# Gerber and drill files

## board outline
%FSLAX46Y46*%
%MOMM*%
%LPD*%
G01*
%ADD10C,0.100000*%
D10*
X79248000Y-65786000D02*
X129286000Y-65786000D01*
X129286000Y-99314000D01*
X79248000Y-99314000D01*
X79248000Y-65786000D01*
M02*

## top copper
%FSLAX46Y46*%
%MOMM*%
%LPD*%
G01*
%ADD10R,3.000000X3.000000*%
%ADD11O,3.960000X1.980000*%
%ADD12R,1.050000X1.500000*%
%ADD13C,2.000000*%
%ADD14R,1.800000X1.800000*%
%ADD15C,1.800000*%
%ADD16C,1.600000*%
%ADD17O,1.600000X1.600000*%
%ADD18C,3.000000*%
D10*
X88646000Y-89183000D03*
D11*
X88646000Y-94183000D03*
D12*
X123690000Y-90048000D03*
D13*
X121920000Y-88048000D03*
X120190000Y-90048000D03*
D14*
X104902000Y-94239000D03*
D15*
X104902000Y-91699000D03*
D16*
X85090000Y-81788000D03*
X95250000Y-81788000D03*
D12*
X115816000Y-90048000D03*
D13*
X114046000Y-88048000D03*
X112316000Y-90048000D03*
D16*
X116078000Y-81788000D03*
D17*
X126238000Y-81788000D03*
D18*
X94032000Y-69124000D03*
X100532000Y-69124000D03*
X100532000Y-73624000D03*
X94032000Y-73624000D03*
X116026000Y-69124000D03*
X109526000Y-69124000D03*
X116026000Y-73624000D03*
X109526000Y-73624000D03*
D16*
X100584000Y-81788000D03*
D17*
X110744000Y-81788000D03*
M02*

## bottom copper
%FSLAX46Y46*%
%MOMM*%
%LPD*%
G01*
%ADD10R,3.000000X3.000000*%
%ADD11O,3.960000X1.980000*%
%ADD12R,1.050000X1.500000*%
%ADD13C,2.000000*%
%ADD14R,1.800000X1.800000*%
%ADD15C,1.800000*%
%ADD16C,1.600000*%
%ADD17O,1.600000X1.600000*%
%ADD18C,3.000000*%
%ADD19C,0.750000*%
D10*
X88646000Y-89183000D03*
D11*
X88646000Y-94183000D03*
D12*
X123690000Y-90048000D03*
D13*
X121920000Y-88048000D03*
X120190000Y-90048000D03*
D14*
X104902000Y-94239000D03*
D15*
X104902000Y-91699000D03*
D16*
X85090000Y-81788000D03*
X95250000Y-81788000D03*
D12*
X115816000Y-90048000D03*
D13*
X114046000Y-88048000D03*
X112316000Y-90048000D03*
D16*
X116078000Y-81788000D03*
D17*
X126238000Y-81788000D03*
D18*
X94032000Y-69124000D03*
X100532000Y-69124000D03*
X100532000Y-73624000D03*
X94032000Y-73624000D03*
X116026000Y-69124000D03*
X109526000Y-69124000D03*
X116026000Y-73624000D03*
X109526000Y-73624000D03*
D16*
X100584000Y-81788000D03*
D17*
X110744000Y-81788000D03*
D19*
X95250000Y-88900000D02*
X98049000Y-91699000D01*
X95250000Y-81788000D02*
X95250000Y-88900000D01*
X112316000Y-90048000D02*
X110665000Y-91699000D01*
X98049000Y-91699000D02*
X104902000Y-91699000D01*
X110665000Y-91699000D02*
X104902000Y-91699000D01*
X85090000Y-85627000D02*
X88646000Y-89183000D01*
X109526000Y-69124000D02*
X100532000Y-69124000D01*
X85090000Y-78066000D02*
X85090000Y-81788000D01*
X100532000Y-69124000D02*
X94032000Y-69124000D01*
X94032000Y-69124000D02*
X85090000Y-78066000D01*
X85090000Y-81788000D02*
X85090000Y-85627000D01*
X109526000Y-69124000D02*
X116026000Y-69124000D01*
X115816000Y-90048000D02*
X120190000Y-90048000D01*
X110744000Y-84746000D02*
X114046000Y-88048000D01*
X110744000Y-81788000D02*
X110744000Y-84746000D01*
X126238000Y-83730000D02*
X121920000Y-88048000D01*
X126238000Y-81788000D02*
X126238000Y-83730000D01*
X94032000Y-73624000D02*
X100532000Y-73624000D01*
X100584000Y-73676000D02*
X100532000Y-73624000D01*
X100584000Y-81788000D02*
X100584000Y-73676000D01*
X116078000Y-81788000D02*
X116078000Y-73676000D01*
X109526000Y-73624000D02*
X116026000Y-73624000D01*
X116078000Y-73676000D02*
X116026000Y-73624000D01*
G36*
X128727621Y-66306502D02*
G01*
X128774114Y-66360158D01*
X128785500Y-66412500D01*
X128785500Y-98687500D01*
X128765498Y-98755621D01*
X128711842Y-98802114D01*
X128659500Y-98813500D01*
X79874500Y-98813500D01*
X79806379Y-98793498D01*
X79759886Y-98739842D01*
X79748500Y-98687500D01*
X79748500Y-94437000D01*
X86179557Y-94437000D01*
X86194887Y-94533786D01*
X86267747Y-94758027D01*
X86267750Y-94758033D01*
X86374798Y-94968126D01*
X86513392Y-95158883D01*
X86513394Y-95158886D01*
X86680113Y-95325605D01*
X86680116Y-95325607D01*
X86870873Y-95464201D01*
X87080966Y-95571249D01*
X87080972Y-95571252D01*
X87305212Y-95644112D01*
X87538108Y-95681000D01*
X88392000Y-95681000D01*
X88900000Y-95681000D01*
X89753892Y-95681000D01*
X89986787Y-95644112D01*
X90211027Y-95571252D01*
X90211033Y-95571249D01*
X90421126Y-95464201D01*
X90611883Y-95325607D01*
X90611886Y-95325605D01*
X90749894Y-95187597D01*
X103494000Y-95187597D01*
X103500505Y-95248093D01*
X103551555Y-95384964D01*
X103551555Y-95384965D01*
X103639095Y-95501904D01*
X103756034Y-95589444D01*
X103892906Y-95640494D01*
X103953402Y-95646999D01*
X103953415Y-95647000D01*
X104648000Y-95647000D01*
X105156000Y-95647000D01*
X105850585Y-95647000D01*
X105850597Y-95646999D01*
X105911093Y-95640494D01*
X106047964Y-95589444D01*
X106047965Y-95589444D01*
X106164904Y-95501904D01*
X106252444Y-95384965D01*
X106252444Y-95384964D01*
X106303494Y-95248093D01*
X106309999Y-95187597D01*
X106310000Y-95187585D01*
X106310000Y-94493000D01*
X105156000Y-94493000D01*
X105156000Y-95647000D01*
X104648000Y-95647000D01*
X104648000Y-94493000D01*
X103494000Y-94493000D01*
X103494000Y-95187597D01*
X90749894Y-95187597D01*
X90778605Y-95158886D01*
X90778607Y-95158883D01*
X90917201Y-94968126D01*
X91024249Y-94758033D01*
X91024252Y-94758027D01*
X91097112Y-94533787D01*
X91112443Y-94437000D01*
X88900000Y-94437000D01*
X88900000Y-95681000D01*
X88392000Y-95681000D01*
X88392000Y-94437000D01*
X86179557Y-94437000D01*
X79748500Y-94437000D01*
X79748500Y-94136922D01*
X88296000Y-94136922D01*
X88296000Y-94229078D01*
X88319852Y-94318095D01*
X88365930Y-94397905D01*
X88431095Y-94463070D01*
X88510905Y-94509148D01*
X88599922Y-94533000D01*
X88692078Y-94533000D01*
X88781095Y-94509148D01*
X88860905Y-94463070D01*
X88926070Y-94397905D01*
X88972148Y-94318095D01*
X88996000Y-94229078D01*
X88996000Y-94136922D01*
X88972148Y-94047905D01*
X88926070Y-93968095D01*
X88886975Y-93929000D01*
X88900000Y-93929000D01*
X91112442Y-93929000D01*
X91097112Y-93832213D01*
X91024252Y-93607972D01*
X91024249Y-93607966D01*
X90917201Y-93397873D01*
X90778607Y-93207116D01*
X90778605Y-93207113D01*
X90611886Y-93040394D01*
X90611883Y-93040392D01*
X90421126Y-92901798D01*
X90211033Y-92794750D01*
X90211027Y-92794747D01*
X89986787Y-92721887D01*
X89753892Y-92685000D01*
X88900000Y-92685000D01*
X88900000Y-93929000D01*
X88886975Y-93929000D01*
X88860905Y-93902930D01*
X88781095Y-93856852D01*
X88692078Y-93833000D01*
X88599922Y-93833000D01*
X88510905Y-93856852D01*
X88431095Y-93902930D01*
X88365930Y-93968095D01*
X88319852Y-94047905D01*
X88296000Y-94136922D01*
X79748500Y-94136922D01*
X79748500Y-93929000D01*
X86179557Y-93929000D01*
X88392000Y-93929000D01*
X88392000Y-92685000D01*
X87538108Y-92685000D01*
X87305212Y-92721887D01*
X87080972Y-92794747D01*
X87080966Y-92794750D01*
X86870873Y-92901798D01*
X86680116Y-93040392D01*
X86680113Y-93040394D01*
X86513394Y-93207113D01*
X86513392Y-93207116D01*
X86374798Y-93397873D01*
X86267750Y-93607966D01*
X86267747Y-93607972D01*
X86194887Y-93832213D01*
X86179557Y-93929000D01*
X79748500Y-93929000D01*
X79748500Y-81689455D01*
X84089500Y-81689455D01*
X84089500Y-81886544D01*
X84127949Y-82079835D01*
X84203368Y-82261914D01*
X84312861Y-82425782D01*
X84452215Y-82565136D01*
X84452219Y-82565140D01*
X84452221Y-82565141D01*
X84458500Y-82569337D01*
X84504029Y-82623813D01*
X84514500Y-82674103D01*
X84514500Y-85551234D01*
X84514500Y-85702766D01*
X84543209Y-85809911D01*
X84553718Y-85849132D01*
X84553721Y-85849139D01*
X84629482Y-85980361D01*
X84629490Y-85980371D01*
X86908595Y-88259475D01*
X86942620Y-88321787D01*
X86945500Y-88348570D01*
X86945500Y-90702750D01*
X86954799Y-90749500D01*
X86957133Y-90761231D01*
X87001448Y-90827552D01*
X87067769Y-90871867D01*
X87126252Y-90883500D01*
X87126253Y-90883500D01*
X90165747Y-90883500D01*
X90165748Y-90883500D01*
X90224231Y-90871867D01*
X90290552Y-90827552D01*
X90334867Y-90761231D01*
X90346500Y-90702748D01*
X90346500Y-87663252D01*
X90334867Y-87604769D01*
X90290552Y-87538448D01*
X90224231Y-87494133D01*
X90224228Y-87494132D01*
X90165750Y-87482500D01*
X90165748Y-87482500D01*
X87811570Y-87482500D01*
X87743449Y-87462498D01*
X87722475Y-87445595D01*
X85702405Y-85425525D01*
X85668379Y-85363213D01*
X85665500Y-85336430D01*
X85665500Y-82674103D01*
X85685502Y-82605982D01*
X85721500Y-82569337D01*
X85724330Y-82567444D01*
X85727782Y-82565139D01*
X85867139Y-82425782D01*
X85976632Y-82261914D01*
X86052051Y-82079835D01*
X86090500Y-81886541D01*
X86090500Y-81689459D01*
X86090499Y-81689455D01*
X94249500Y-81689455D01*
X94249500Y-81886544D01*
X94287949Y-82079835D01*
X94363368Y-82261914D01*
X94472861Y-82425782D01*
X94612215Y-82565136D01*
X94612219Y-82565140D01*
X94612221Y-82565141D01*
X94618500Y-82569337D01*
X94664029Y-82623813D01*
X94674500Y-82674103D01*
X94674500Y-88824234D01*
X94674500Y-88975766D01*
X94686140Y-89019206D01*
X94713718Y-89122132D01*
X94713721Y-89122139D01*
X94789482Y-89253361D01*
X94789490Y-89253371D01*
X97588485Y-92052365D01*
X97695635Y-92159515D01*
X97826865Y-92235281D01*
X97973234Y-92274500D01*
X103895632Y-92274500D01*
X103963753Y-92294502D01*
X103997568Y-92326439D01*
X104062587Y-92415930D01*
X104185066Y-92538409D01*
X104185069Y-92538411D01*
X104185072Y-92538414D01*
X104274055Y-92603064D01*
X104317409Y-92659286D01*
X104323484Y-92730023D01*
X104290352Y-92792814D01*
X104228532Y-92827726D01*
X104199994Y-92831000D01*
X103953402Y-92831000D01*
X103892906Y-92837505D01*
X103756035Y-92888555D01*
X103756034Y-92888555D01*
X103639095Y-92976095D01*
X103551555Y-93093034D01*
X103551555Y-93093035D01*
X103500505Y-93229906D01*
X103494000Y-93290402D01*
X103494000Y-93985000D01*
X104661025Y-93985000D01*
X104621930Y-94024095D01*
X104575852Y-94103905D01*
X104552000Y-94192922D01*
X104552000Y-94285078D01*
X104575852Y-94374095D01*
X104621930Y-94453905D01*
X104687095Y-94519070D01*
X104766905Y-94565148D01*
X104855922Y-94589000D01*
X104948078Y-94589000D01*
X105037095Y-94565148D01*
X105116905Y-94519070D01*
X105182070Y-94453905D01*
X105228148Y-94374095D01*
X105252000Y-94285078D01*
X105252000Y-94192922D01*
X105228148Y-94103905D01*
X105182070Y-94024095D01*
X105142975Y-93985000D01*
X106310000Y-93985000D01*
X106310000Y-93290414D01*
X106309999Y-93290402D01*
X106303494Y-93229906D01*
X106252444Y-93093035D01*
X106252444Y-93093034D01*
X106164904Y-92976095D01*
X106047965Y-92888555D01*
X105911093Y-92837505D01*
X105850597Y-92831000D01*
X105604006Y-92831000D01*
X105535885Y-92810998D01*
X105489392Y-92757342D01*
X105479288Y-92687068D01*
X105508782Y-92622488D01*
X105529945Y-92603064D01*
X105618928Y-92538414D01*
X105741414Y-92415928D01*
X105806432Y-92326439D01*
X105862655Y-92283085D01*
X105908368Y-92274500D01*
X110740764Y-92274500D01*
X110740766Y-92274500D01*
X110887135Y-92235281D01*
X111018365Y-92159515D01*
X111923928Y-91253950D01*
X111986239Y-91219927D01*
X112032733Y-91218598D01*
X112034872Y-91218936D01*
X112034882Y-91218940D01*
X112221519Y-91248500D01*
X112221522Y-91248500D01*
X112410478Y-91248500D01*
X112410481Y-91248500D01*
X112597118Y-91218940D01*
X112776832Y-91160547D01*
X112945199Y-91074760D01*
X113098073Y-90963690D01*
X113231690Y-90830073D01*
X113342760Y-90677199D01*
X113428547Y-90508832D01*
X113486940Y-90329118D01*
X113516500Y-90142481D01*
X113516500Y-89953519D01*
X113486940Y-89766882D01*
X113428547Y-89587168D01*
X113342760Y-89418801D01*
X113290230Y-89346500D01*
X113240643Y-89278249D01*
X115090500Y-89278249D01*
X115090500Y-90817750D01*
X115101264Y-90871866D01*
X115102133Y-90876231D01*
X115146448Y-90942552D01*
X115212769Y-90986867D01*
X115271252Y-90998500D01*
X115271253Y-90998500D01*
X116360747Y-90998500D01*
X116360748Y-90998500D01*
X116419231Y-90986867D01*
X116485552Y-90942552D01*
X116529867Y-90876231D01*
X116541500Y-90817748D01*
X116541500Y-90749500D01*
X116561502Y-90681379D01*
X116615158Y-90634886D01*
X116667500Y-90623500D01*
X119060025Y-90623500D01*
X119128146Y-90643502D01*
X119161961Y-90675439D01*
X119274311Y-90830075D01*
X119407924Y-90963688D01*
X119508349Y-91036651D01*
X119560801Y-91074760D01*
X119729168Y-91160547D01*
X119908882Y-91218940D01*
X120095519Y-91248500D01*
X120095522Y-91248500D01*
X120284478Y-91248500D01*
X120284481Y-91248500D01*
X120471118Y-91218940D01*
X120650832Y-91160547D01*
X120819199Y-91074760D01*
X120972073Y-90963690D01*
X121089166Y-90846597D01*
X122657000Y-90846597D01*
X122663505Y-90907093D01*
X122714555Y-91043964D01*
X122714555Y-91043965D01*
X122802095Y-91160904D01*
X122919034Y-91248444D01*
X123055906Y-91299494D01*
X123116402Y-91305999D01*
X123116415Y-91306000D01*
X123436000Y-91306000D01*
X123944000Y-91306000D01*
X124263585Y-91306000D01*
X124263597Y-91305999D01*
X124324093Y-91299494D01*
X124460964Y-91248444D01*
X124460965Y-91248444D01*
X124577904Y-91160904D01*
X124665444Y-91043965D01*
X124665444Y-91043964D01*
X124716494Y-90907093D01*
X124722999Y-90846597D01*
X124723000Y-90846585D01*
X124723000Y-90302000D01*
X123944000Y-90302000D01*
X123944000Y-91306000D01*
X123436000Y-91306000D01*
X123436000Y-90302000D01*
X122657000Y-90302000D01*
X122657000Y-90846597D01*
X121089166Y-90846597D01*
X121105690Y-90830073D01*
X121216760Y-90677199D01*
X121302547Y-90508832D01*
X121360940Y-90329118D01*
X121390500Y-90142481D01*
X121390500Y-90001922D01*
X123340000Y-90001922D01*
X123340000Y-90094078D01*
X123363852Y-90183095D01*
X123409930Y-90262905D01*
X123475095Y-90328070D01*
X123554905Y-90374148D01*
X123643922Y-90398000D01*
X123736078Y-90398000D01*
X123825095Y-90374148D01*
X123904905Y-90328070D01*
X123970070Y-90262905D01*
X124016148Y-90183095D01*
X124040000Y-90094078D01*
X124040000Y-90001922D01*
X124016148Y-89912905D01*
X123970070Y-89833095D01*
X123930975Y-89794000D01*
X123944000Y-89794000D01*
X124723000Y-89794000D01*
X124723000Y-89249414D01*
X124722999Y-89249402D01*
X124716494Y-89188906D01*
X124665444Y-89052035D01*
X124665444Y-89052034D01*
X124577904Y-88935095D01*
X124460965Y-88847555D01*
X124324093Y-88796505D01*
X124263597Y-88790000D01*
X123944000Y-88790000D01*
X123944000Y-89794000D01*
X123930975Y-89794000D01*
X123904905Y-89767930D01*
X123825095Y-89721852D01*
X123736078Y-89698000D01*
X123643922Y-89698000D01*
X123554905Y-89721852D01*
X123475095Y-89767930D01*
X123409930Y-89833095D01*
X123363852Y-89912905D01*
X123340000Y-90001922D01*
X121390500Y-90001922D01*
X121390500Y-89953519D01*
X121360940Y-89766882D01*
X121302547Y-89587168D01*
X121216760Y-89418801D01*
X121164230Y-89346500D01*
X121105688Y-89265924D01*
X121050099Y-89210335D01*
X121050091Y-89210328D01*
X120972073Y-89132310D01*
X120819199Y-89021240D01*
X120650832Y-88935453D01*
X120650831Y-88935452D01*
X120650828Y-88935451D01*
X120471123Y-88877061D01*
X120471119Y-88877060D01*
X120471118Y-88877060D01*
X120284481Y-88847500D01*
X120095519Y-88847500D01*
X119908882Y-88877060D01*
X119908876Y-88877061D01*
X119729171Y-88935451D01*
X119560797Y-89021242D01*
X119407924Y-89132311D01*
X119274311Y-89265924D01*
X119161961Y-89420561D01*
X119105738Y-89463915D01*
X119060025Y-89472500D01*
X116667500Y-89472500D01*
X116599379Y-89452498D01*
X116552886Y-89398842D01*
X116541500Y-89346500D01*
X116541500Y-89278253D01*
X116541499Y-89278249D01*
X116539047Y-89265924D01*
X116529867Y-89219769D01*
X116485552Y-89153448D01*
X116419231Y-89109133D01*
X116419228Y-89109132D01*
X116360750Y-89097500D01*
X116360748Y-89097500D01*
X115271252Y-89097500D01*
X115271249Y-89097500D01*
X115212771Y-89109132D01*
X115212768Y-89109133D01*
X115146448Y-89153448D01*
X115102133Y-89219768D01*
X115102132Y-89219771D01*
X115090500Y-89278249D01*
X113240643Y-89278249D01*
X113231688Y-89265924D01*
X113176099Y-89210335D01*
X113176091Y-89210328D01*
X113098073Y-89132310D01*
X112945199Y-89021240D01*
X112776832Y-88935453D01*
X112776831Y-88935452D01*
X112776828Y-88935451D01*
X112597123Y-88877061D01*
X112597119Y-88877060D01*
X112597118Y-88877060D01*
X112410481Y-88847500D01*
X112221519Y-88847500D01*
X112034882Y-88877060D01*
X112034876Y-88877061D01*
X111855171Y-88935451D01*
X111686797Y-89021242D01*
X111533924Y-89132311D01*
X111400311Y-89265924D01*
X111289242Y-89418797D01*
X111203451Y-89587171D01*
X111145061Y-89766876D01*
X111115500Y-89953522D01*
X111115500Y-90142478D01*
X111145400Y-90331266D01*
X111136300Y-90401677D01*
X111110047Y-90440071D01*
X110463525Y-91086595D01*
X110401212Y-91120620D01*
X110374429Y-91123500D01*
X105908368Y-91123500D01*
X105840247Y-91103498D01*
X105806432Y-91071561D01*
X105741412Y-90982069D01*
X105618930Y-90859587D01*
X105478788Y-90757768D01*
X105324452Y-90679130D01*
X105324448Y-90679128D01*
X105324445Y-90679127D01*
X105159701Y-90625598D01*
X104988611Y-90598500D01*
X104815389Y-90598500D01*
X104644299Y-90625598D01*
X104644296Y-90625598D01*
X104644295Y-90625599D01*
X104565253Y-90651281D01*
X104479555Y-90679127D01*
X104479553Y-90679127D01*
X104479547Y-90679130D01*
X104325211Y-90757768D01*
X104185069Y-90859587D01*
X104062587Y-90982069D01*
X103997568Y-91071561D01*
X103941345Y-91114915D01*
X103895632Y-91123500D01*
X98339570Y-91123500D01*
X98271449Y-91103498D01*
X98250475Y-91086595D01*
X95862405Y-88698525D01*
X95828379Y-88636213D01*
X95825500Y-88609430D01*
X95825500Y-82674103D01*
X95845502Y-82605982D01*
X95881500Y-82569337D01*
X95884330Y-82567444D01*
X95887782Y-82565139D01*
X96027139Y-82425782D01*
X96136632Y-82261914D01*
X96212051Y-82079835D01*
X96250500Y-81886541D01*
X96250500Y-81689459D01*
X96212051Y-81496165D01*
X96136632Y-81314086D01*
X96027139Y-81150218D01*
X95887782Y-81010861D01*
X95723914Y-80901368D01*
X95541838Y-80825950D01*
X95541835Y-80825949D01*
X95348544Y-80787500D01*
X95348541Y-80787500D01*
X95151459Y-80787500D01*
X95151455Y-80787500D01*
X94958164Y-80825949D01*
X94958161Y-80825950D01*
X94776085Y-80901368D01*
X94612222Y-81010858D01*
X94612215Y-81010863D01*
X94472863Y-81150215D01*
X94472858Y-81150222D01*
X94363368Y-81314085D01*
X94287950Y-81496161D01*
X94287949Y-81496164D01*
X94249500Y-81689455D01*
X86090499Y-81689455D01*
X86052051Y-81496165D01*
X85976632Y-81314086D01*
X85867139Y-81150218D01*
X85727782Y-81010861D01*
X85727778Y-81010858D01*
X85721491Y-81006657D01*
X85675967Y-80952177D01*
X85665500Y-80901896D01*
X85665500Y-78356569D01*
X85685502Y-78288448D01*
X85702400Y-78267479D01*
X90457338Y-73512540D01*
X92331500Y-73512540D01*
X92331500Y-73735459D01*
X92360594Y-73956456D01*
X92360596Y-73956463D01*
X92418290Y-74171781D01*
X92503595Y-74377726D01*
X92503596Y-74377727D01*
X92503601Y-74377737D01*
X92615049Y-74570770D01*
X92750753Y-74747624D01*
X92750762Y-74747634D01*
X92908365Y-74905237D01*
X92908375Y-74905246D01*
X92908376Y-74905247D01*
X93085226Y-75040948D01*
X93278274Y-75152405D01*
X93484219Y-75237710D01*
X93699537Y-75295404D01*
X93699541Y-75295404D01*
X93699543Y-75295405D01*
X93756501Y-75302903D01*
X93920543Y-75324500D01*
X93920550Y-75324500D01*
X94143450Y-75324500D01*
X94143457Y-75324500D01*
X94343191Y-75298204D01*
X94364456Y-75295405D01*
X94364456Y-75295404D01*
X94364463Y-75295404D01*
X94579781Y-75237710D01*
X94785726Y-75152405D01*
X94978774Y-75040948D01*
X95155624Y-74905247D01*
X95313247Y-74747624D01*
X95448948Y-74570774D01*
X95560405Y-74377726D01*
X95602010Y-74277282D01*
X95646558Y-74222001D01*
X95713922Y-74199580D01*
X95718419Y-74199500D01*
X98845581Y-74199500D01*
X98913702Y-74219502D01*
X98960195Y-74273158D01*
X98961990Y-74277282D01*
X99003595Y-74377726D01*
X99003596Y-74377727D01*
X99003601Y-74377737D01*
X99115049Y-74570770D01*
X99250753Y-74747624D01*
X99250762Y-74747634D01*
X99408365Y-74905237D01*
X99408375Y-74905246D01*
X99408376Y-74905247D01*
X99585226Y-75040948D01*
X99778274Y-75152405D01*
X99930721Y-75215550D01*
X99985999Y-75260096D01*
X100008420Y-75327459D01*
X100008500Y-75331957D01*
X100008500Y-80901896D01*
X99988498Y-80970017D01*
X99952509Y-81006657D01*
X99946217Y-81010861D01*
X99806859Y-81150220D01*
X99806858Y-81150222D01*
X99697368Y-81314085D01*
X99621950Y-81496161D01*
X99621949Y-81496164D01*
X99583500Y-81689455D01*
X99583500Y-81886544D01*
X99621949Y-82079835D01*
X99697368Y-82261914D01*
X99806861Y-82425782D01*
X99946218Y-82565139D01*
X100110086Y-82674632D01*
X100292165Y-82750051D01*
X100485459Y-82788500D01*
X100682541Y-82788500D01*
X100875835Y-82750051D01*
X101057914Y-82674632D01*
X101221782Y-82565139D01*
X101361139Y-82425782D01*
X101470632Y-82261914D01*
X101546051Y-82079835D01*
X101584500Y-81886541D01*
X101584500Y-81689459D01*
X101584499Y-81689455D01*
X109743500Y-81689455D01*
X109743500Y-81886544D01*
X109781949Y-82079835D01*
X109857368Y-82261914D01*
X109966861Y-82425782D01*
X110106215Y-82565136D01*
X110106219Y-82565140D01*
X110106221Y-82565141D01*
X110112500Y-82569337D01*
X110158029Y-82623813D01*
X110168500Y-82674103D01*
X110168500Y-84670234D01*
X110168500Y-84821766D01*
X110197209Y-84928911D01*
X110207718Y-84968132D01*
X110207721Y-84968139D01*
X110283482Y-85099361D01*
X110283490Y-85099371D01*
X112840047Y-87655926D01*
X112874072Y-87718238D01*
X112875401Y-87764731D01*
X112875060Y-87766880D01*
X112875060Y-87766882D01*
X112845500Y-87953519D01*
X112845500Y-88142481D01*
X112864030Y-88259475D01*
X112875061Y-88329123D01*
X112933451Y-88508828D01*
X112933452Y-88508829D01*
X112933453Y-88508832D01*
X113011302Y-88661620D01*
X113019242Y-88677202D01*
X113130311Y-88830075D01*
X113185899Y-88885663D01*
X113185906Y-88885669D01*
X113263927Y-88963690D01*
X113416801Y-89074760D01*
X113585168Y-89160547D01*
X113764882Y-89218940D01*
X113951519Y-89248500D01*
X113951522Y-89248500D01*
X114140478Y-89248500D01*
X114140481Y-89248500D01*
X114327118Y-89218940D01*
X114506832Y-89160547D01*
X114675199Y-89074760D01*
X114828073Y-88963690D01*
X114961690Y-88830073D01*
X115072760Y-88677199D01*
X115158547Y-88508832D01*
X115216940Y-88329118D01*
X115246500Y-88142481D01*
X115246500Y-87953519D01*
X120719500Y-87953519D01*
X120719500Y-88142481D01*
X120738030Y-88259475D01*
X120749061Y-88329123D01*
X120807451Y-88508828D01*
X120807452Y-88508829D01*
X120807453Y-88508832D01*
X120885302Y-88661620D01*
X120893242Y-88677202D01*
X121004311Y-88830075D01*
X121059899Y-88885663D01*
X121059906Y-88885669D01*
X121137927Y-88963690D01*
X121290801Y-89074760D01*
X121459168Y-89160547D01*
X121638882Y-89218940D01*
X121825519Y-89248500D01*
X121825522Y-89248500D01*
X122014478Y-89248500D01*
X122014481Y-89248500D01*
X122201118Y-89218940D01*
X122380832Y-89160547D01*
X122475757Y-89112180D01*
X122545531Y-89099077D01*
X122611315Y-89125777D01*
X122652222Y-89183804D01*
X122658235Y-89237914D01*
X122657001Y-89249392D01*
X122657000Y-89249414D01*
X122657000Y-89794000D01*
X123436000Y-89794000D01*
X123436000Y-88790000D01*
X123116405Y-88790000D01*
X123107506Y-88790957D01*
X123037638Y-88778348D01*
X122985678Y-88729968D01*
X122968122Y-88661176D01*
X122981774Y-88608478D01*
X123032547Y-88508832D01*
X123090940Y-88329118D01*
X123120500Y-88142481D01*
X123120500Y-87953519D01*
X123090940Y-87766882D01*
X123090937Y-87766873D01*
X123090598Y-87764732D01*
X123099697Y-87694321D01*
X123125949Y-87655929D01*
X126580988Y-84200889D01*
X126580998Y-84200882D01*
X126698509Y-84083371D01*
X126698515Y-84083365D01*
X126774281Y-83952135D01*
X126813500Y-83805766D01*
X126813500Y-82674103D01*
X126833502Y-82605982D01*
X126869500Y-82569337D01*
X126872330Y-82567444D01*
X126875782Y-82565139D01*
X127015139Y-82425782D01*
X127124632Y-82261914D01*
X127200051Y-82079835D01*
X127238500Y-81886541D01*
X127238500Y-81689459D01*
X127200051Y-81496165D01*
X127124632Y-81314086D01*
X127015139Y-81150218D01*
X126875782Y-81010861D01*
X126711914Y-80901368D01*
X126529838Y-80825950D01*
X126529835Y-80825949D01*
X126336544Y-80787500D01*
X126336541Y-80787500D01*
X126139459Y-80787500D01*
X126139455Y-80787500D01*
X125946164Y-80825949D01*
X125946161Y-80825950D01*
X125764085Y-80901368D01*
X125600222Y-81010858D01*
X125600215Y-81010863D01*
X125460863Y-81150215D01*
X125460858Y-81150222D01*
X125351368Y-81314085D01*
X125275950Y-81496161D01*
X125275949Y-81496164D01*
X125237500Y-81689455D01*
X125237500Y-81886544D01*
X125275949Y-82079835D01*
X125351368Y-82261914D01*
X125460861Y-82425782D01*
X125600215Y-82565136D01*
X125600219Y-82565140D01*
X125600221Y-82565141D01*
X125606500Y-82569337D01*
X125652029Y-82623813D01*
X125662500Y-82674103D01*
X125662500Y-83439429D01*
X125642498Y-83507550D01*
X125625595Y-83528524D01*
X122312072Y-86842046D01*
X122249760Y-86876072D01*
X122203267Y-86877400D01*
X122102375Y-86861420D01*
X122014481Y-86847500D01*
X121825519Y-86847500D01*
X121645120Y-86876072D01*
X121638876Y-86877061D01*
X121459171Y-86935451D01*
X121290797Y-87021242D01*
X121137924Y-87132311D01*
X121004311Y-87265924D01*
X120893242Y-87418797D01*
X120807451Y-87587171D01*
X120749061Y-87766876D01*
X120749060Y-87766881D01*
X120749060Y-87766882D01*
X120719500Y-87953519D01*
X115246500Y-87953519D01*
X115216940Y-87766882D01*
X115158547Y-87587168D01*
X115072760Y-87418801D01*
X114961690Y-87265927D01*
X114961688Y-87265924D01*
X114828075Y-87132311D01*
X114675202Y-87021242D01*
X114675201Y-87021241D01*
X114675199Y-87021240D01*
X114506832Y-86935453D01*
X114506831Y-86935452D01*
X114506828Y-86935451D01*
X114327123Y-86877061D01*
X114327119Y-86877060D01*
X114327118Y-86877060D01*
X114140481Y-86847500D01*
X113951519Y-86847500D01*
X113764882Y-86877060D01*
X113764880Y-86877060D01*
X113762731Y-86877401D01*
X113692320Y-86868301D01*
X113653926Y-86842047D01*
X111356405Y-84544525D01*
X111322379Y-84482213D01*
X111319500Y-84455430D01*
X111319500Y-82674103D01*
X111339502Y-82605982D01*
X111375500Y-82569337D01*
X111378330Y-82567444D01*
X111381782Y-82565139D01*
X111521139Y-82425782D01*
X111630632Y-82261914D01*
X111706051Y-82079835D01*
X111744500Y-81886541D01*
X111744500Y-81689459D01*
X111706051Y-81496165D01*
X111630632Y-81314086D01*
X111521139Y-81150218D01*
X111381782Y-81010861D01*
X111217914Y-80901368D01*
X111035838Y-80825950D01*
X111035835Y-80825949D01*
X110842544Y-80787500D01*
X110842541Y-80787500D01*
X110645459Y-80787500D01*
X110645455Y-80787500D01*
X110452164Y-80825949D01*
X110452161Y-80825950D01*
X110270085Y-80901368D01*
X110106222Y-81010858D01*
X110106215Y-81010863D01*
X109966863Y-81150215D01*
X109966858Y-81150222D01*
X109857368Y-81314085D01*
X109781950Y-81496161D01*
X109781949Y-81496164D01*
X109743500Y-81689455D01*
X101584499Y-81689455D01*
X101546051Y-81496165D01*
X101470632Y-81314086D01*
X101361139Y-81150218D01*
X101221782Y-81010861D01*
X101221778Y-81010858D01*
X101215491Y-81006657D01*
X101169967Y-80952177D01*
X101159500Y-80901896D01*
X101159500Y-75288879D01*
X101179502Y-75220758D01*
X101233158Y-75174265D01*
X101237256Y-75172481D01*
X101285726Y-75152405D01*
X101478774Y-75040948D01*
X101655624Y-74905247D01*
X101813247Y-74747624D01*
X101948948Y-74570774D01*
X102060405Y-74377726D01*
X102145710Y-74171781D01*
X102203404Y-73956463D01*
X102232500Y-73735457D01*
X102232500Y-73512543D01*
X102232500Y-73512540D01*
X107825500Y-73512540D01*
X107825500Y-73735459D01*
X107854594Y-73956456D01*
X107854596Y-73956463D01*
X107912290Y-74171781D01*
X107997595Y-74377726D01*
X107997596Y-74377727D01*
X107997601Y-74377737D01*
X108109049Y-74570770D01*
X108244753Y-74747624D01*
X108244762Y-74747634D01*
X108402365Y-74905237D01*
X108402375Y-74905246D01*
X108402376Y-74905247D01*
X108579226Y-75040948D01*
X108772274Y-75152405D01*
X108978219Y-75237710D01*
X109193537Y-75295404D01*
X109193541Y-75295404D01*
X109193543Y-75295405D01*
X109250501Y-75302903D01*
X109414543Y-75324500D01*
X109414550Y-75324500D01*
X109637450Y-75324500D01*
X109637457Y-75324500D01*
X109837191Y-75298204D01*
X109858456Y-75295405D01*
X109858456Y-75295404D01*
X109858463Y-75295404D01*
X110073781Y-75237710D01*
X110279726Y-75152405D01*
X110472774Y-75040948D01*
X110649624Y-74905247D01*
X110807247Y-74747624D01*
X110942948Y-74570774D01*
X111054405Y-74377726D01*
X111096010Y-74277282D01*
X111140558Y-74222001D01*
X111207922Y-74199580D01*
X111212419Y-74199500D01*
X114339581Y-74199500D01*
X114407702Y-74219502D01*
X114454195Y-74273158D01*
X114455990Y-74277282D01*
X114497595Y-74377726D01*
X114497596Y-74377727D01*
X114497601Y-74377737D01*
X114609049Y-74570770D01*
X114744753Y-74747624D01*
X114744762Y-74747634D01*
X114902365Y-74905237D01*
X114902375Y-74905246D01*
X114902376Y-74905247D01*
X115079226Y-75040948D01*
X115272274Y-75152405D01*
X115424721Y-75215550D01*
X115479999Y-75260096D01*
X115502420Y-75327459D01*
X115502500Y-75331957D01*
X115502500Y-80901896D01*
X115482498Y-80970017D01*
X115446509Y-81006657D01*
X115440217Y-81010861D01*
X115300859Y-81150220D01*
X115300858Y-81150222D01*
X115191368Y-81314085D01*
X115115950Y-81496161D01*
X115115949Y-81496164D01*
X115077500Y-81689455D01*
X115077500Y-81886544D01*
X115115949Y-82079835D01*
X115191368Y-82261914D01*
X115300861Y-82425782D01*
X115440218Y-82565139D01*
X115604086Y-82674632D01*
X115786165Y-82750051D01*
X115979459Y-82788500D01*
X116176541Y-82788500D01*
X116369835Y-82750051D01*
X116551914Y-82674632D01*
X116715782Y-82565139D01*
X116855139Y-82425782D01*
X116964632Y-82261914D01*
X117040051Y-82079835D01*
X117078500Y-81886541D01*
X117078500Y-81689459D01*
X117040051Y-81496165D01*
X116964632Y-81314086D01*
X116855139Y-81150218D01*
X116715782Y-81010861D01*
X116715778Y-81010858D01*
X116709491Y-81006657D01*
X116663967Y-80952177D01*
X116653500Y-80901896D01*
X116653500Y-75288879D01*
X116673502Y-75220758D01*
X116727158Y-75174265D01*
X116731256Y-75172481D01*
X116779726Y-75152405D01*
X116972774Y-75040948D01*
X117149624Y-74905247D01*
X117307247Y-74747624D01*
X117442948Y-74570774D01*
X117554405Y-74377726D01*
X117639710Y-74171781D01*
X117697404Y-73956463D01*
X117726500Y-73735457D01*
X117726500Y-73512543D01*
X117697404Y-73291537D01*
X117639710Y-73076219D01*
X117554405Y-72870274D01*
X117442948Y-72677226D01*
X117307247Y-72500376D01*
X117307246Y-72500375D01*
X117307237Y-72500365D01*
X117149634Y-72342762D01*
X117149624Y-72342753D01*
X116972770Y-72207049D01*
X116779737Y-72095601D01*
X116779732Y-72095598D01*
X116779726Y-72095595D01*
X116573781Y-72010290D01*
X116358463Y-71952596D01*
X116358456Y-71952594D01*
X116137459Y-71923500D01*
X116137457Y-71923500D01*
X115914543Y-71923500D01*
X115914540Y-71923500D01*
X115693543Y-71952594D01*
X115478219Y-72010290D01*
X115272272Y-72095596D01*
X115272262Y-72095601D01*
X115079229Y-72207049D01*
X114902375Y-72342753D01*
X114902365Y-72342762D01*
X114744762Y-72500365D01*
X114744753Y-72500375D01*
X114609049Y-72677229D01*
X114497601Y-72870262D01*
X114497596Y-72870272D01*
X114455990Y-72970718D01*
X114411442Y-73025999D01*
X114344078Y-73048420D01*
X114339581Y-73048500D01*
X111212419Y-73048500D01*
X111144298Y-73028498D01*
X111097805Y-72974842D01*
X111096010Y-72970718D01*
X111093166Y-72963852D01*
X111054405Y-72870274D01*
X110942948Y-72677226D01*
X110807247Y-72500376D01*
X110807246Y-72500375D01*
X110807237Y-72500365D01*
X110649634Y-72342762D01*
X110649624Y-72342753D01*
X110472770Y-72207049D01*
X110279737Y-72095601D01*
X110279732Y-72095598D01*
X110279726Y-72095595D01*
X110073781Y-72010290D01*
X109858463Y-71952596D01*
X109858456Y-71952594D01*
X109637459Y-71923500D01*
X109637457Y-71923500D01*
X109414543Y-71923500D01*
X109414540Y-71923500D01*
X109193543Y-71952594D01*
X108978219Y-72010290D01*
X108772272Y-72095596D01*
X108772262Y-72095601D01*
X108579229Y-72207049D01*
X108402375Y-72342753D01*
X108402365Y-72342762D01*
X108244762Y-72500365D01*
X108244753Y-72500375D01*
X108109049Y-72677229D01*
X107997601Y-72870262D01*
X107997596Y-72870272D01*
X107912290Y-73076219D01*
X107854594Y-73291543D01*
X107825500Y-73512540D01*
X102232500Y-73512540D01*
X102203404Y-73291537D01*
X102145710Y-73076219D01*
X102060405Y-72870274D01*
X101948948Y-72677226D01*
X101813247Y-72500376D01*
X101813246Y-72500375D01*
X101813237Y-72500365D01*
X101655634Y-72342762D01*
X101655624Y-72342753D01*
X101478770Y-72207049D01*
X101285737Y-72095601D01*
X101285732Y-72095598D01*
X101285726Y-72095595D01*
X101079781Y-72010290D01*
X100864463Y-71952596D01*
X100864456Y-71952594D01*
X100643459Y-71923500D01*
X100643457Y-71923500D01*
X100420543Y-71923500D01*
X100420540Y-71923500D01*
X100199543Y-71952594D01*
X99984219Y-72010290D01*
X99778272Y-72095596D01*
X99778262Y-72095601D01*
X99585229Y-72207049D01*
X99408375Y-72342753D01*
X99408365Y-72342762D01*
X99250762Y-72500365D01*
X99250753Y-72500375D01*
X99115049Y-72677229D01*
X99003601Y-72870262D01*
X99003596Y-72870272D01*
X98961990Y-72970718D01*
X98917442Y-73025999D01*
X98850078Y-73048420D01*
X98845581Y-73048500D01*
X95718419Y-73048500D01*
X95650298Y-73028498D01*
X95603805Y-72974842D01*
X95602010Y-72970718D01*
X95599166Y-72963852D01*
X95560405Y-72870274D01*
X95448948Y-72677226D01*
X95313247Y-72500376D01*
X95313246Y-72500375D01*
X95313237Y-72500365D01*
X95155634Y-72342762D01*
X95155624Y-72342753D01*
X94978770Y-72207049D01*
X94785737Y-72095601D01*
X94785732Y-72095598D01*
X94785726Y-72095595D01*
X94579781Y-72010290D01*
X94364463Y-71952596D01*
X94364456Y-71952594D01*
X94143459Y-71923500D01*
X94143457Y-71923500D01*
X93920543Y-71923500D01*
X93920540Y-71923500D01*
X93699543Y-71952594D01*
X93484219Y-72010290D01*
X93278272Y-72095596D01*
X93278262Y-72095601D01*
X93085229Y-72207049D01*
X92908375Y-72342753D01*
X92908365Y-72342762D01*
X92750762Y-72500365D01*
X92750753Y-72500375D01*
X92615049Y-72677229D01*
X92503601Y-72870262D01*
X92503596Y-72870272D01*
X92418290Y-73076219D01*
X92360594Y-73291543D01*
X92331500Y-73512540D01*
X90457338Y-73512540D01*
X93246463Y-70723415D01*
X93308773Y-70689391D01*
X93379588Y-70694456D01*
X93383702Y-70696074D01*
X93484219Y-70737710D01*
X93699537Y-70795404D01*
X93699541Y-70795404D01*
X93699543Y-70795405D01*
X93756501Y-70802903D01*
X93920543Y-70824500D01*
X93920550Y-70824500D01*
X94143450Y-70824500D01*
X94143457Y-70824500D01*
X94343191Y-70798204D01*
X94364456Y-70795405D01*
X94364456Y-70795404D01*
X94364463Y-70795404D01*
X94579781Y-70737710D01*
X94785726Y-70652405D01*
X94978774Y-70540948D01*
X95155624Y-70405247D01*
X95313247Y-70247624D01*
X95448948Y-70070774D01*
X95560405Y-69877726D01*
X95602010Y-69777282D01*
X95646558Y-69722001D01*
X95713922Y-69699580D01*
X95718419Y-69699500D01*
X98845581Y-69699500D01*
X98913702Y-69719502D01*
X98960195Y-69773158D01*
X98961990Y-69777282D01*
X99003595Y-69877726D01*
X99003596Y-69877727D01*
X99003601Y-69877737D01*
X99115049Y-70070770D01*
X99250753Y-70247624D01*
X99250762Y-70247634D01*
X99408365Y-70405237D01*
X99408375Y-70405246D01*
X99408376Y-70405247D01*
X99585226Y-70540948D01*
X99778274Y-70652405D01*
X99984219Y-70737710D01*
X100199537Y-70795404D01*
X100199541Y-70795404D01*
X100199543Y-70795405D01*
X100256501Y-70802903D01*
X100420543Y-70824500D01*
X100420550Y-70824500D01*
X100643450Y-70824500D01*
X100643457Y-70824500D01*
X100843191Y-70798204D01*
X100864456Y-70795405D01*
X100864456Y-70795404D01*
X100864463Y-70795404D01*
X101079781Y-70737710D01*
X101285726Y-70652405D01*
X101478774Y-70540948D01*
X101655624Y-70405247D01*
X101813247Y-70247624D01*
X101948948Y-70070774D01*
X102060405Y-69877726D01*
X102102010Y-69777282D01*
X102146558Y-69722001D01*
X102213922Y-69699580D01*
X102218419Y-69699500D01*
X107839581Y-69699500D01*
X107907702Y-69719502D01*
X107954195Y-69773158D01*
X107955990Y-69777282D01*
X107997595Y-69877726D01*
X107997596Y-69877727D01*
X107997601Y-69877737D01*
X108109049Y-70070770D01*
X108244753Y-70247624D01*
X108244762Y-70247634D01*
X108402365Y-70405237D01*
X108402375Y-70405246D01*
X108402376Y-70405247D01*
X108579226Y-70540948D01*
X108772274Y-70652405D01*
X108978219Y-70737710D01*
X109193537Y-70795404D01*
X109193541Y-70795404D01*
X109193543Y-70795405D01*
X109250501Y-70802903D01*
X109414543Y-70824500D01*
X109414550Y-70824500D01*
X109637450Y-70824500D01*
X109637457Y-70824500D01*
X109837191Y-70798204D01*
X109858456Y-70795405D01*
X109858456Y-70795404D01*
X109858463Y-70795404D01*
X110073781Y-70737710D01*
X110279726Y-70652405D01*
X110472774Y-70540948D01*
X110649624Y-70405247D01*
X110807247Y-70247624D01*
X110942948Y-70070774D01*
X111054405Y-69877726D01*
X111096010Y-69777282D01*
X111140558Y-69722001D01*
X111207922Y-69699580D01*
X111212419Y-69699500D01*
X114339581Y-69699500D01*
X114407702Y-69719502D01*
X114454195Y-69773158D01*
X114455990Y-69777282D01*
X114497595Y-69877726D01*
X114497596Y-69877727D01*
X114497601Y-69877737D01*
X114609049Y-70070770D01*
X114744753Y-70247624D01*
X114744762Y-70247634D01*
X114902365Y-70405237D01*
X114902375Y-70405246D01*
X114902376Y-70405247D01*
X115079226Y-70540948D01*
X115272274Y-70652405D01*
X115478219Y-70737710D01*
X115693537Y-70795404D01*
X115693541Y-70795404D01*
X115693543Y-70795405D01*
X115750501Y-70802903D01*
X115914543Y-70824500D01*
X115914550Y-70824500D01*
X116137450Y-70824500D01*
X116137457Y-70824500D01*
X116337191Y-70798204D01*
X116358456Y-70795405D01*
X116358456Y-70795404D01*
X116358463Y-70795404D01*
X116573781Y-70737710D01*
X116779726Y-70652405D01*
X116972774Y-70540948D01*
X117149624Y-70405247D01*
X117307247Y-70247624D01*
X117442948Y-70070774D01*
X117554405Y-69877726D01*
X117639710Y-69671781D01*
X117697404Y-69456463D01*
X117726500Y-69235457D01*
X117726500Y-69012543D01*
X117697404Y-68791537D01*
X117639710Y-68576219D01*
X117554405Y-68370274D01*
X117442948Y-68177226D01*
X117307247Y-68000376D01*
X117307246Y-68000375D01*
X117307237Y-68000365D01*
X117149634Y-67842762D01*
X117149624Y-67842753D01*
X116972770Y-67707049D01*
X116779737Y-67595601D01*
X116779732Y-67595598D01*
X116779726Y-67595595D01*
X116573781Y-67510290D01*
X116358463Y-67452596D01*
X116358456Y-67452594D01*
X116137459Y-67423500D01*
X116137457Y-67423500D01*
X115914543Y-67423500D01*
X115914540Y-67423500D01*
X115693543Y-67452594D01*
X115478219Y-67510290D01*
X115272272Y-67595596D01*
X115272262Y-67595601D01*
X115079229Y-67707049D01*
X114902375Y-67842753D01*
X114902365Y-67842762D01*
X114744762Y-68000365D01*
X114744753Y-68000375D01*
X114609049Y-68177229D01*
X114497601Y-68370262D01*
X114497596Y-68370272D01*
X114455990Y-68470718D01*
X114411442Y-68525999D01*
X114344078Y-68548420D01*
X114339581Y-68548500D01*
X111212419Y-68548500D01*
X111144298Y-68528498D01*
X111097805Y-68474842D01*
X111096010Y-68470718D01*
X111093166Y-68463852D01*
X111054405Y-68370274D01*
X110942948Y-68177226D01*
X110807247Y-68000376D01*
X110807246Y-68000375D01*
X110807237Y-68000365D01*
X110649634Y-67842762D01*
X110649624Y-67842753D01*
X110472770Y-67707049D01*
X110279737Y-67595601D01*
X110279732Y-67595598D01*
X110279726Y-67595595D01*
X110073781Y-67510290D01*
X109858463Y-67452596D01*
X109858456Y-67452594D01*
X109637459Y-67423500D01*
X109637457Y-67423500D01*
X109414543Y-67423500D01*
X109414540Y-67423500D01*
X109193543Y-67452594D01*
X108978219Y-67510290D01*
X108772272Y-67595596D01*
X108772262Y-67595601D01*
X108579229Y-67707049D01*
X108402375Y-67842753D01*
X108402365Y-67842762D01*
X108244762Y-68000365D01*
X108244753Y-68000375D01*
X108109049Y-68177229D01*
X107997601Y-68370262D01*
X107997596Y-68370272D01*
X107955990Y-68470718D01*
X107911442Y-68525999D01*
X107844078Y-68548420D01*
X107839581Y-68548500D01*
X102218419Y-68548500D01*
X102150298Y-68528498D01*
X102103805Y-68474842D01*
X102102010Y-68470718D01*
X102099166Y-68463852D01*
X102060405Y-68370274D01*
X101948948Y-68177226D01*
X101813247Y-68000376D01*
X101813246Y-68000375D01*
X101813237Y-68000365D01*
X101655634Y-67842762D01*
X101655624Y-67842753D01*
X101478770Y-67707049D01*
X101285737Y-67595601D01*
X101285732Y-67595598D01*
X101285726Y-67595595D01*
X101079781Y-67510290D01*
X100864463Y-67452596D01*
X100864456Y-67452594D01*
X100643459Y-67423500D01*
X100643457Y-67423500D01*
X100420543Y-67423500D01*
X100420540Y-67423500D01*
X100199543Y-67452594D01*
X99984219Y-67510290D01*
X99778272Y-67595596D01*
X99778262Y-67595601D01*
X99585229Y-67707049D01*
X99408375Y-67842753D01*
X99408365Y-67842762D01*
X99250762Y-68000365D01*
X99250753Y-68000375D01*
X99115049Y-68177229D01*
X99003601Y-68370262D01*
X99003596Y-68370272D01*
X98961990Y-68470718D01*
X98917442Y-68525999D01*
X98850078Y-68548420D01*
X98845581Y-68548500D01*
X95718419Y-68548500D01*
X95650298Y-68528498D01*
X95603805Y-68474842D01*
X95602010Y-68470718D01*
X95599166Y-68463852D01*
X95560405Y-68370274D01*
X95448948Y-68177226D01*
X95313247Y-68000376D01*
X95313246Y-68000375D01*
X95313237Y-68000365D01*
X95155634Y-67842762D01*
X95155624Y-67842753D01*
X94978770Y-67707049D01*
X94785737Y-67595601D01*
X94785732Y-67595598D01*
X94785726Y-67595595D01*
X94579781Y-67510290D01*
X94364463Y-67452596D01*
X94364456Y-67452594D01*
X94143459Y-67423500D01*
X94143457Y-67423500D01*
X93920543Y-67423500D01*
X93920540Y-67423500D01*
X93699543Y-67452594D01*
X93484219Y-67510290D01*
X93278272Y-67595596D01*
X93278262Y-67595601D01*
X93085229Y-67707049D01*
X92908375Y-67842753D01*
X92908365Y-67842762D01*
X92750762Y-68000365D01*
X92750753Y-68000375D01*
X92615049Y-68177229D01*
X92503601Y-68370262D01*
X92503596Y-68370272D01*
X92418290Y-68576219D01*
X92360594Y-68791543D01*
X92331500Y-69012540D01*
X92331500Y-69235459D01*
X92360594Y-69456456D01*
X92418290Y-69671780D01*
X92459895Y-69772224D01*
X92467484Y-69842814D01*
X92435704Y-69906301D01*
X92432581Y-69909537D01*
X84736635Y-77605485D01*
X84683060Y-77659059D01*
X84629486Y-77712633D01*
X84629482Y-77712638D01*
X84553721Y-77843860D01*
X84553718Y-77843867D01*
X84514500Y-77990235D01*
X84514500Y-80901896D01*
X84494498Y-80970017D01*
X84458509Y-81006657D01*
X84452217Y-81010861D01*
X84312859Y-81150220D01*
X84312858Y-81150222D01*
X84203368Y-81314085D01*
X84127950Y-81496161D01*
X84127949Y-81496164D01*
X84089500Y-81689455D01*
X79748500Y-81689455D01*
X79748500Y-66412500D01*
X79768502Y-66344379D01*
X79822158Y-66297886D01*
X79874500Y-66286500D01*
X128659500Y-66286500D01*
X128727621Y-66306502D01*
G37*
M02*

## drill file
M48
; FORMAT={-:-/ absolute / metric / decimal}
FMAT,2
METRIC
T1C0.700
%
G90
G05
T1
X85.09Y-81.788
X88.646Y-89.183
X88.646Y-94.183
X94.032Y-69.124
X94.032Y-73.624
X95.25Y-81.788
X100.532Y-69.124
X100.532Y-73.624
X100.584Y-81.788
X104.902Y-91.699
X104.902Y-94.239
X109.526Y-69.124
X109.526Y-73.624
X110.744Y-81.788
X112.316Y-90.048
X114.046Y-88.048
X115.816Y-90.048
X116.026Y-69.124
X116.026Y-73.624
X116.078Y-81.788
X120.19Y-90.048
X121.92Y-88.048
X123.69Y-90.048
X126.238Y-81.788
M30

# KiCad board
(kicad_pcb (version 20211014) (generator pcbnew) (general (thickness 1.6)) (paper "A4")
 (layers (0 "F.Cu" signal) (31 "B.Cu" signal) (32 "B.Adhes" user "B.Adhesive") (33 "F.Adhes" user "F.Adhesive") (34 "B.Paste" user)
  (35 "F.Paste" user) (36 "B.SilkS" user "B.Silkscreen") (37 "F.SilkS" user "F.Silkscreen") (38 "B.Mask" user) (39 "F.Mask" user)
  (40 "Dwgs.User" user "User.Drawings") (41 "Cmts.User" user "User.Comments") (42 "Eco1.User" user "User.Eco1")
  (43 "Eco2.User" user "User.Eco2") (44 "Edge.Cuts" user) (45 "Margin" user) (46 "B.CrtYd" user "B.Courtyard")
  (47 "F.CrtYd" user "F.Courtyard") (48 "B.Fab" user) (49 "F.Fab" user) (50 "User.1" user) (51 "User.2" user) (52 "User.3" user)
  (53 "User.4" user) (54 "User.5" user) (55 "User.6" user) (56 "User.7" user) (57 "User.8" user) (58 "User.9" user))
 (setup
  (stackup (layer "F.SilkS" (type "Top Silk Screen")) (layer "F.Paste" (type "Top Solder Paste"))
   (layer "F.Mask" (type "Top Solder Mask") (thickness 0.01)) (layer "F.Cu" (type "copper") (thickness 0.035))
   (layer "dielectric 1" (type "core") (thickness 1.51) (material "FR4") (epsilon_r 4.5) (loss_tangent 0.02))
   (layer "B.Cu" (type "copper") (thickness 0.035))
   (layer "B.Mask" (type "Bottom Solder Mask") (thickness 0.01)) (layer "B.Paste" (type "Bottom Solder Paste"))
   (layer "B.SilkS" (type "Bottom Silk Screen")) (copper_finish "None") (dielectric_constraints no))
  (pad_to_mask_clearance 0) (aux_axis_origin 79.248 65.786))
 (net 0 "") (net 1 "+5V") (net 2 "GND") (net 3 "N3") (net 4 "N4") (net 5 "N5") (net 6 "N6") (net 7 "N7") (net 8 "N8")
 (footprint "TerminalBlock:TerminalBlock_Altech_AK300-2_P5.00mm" (layer "F.Cu") (at 88.646 89.183 -90)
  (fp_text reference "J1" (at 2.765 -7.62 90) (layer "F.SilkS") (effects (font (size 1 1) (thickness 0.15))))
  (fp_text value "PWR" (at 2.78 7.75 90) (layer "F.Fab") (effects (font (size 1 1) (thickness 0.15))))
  (pad "1" thru_hole rect (at 0 0 270) (size 3 3) (drill 0.7) (layers *.Cu *.Mask) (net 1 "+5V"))
  (pad "2" thru_hole oval (at 5 0 270) (size 1.98 3.96) (drill 0.7) (layers *.Cu *.Mask) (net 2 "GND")))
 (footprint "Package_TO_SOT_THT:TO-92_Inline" (layer "F.Cu") (at 123.19 89.048 180)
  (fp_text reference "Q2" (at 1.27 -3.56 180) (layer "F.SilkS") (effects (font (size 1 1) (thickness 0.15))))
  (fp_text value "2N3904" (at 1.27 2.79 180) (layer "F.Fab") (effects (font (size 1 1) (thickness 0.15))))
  (pad "1" thru_hole rect (at -0.5 -1 180) (size 1.05 1.5) (drill 0.7) (layers *.Cu *.Mask) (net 2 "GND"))
  (pad "2" thru_hole circle (at 1.27 1 180) (size 2 2) (drill 0.7) (layers *.Cu *.Mask) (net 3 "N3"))
  (pad "3" thru_hole circle (at 3 -1 180) (size 2 2) (drill 0.7) (layers *.Cu *.Mask) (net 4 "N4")))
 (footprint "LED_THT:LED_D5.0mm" (layer "F.Cu") (at 104.902 94.239 90)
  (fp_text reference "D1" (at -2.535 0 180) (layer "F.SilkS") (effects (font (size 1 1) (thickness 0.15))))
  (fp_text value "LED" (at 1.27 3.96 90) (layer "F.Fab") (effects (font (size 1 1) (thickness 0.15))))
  (pad "1" thru_hole rect (at 0 0 90) (size 1.8 1.8) (drill 0.7) (layers *.Cu *.Mask) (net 2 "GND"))
  (pad "2" thru_hole circle (at 2.54 0 90) (size 1.8 1.8) (drill 0.7) (layers *.Cu *.Mask) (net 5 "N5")))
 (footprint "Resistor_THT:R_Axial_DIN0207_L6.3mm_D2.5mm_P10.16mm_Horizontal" (layer "F.Cu") (at 85.09 81.788)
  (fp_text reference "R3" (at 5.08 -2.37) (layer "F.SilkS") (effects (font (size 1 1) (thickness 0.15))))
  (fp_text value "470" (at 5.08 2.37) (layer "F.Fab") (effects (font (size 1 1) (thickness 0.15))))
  (pad "1" thru_hole circle (at 0 0) (size 1.6 1.6) (drill 0.7) (layers *.Cu *.Mask) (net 1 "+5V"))
  (pad "2" thru_hole circle (at 10.16 0) (size 1.6 1.6) (drill 0.7) (layers *.Cu *.Mask) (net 5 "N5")))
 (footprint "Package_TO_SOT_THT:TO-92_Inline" (layer "F.Cu") (at 115.316 89.048 180)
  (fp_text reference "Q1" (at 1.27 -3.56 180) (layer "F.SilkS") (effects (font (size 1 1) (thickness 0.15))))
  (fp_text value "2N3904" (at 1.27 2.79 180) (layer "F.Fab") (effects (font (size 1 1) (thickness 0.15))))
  (pad "1" thru_hole rect (at -0.5 -1 180) (size 1.05 1.5) (drill 0.7) (layers *.Cu *.Mask) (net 4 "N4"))
  (pad "2" thru_hole circle (at 1.27 1 180) (size 2 2) (drill 0.7) (layers *.Cu *.Mask) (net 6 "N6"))
  (pad "3" thru_hole circle (at 3 -1 180) (size 2 2) (drill 0.7) (layers *.Cu *.Mask) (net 5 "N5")))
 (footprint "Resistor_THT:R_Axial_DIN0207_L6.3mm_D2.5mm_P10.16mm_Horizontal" (layer "F.Cu") (at 116.078 81.788)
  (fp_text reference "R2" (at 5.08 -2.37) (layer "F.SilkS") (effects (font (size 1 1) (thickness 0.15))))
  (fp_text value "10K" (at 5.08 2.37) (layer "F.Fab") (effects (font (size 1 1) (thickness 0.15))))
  (pad "1" thru_hole circle (at 0 0) (size 1.6 1.6) (drill 0.7) (layers *.Cu *.Mask) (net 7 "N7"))
  (pad "2" thru_hole oval (at 10.16 0) (size 1.6 1.6) (drill 0.7) (layers *.Cu *.Mask) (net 3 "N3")))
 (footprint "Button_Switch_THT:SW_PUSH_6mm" (layer "F.Cu") (at 94.032 69.124)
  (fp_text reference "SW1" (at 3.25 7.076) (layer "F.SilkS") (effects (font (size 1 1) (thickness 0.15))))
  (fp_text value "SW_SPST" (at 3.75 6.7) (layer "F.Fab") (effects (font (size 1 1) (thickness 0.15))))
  (pad "1" thru_hole circle (at 0 0 90) (size 3 3) (drill 0.7) (layers *.Cu *.Mask) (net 1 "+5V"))
  (pad "1" thru_hole circle (at 6.5 0 90) (size 3 3) (drill 0.7) (layers *.Cu *.Mask) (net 1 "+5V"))
  (pad "2" thru_hole circle (at 6.5 4.5 90) (size 3 3) (drill 0.7) (layers *.Cu *.Mask) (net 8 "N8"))
  (pad "2" thru_hole circle (at 0 4.5 90) (size 3 3) (drill 0.7) (layers *.Cu *.Mask) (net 8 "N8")))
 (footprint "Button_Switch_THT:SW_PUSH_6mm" (layer "F.Cu") (at 109.526 69.124)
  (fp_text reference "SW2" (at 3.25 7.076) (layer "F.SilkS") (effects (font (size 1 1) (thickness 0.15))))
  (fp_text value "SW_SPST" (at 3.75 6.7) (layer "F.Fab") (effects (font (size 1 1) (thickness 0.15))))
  (pad "1" thru_hole circle (at 6.5 0 90) (size 3 3) (drill 0.7) (layers *.Cu *.Mask) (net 1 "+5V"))
  (pad "1" thru_hole circle (at 0 0 90) (size 3 3) (drill 0.7) (layers *.Cu *.Mask) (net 1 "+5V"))
  (pad "2" thru_hole circle (at 6.5 4.5 90) (size 3 3) (drill 0.7) (layers *.Cu *.Mask) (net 7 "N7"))
  (pad "2" thru_hole circle (at 0 4.5 90) (size 3 3) (drill 0.7) (layers *.Cu *.Mask) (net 7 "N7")))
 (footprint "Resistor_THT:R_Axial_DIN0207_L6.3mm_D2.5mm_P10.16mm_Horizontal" (layer "F.Cu") (at 100.584 81.788)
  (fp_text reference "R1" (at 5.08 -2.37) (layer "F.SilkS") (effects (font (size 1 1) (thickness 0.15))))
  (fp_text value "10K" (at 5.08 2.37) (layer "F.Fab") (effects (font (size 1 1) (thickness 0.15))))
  (pad "1" thru_hole circle (at 0 0) (size 1.6 1.6) (drill 0.7) (layers *.Cu *.Mask) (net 8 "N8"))
  (pad "2" thru_hole oval (at 10.16 0) (size 1.6 1.6) (drill 0.7) (layers *.Cu *.Mask) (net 6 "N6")))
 (gr_rect (start 79.248 65.786) (end 129.286 99.314) (layer "Edge.Cuts") (width 0.1) (fill none))
 (segment (start 95.25 88.9) (end 98.049 91.699) (width 0.75) (layer "B.Cu") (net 5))
 (segment (start 95.25 81.788) (end 95.25 88.9) (width 0.75) (layer "B.Cu") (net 5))
 (segment (start 112.316 90.048) (end 110.665 91.699) (width 0.75) (layer "B.Cu") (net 5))
 (segment (start 98.049 91.699) (end 104.902 91.699) (width 0.75) (layer "B.Cu") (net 5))
 (segment (start 110.665 91.699) (end 104.902 91.699) (width 0.75) (layer "B.Cu") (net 5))
 (segment (start 85.09 85.627) (end 88.646 89.183) (width 0.75) (layer "B.Cu") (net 1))
 (segment (start 109.526 69.124) (end 100.532 69.124) (width 0.75) (layer "B.Cu") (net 1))
 (segment (start 85.09 78.066) (end 85.09 81.788) (width 0.75) (layer "B.Cu") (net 1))
 (segment (start 100.532 69.124) (end 94.032 69.124) (width 0.75) (layer "B.Cu") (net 1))
 (segment (start 94.032 69.124) (end 85.09 78.066) (width 0.75) (layer "B.Cu") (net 1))
 (segment (start 85.09 81.788) (end 85.09 85.627) (width 0.75) (layer "B.Cu") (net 1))
 (segment (start 109.526 69.124) (end 116.026 69.124) (width 0.75) (layer "B.Cu") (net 1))
 (segment (start 115.816 90.048) (end 120.19 90.048) (width 0.75) (layer "B.Cu") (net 4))
 (segment (start 110.744 84.746) (end 114.046 88.048) (width 0.75) (layer "B.Cu") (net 6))
 (segment (start 110.744 81.788) (end 110.744 84.746) (width 0.75) (layer "B.Cu") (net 6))
 (segment (start 126.238 83.73) (end 121.92 88.048) (width 0.75) (layer "B.Cu") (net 3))
 (segment (start 126.238 81.788) (end 126.238 83.73) (width 0.75) (layer "B.Cu") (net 3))
 (segment (start 94.032 73.624) (end 100.532 73.624) (width 0.75) (layer "B.Cu") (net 8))
 (segment (start 100.584 73.676) (end 100.532 73.624) (width 0.75) (layer "B.Cu") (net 8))
 (segment (start 100.584 81.788) (end 100.584 73.676) (width 0.75) (layer "B.Cu") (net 8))
 (segment (start 116.078 81.788) (end 116.078 73.676) (width 0.75) (layer "B.Cu") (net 7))
 (segment (start 109.526 73.624) (end 116.026 73.624) (width 0.75) (layer "B.Cu") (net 7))
 (segment (start 116.078 73.676) (end 116.026 73.624) (width 0.75) (layer "B.Cu") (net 7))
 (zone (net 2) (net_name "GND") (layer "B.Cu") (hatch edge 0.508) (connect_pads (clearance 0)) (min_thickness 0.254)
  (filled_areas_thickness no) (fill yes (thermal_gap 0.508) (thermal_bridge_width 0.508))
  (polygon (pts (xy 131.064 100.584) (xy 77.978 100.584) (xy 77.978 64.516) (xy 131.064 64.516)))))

